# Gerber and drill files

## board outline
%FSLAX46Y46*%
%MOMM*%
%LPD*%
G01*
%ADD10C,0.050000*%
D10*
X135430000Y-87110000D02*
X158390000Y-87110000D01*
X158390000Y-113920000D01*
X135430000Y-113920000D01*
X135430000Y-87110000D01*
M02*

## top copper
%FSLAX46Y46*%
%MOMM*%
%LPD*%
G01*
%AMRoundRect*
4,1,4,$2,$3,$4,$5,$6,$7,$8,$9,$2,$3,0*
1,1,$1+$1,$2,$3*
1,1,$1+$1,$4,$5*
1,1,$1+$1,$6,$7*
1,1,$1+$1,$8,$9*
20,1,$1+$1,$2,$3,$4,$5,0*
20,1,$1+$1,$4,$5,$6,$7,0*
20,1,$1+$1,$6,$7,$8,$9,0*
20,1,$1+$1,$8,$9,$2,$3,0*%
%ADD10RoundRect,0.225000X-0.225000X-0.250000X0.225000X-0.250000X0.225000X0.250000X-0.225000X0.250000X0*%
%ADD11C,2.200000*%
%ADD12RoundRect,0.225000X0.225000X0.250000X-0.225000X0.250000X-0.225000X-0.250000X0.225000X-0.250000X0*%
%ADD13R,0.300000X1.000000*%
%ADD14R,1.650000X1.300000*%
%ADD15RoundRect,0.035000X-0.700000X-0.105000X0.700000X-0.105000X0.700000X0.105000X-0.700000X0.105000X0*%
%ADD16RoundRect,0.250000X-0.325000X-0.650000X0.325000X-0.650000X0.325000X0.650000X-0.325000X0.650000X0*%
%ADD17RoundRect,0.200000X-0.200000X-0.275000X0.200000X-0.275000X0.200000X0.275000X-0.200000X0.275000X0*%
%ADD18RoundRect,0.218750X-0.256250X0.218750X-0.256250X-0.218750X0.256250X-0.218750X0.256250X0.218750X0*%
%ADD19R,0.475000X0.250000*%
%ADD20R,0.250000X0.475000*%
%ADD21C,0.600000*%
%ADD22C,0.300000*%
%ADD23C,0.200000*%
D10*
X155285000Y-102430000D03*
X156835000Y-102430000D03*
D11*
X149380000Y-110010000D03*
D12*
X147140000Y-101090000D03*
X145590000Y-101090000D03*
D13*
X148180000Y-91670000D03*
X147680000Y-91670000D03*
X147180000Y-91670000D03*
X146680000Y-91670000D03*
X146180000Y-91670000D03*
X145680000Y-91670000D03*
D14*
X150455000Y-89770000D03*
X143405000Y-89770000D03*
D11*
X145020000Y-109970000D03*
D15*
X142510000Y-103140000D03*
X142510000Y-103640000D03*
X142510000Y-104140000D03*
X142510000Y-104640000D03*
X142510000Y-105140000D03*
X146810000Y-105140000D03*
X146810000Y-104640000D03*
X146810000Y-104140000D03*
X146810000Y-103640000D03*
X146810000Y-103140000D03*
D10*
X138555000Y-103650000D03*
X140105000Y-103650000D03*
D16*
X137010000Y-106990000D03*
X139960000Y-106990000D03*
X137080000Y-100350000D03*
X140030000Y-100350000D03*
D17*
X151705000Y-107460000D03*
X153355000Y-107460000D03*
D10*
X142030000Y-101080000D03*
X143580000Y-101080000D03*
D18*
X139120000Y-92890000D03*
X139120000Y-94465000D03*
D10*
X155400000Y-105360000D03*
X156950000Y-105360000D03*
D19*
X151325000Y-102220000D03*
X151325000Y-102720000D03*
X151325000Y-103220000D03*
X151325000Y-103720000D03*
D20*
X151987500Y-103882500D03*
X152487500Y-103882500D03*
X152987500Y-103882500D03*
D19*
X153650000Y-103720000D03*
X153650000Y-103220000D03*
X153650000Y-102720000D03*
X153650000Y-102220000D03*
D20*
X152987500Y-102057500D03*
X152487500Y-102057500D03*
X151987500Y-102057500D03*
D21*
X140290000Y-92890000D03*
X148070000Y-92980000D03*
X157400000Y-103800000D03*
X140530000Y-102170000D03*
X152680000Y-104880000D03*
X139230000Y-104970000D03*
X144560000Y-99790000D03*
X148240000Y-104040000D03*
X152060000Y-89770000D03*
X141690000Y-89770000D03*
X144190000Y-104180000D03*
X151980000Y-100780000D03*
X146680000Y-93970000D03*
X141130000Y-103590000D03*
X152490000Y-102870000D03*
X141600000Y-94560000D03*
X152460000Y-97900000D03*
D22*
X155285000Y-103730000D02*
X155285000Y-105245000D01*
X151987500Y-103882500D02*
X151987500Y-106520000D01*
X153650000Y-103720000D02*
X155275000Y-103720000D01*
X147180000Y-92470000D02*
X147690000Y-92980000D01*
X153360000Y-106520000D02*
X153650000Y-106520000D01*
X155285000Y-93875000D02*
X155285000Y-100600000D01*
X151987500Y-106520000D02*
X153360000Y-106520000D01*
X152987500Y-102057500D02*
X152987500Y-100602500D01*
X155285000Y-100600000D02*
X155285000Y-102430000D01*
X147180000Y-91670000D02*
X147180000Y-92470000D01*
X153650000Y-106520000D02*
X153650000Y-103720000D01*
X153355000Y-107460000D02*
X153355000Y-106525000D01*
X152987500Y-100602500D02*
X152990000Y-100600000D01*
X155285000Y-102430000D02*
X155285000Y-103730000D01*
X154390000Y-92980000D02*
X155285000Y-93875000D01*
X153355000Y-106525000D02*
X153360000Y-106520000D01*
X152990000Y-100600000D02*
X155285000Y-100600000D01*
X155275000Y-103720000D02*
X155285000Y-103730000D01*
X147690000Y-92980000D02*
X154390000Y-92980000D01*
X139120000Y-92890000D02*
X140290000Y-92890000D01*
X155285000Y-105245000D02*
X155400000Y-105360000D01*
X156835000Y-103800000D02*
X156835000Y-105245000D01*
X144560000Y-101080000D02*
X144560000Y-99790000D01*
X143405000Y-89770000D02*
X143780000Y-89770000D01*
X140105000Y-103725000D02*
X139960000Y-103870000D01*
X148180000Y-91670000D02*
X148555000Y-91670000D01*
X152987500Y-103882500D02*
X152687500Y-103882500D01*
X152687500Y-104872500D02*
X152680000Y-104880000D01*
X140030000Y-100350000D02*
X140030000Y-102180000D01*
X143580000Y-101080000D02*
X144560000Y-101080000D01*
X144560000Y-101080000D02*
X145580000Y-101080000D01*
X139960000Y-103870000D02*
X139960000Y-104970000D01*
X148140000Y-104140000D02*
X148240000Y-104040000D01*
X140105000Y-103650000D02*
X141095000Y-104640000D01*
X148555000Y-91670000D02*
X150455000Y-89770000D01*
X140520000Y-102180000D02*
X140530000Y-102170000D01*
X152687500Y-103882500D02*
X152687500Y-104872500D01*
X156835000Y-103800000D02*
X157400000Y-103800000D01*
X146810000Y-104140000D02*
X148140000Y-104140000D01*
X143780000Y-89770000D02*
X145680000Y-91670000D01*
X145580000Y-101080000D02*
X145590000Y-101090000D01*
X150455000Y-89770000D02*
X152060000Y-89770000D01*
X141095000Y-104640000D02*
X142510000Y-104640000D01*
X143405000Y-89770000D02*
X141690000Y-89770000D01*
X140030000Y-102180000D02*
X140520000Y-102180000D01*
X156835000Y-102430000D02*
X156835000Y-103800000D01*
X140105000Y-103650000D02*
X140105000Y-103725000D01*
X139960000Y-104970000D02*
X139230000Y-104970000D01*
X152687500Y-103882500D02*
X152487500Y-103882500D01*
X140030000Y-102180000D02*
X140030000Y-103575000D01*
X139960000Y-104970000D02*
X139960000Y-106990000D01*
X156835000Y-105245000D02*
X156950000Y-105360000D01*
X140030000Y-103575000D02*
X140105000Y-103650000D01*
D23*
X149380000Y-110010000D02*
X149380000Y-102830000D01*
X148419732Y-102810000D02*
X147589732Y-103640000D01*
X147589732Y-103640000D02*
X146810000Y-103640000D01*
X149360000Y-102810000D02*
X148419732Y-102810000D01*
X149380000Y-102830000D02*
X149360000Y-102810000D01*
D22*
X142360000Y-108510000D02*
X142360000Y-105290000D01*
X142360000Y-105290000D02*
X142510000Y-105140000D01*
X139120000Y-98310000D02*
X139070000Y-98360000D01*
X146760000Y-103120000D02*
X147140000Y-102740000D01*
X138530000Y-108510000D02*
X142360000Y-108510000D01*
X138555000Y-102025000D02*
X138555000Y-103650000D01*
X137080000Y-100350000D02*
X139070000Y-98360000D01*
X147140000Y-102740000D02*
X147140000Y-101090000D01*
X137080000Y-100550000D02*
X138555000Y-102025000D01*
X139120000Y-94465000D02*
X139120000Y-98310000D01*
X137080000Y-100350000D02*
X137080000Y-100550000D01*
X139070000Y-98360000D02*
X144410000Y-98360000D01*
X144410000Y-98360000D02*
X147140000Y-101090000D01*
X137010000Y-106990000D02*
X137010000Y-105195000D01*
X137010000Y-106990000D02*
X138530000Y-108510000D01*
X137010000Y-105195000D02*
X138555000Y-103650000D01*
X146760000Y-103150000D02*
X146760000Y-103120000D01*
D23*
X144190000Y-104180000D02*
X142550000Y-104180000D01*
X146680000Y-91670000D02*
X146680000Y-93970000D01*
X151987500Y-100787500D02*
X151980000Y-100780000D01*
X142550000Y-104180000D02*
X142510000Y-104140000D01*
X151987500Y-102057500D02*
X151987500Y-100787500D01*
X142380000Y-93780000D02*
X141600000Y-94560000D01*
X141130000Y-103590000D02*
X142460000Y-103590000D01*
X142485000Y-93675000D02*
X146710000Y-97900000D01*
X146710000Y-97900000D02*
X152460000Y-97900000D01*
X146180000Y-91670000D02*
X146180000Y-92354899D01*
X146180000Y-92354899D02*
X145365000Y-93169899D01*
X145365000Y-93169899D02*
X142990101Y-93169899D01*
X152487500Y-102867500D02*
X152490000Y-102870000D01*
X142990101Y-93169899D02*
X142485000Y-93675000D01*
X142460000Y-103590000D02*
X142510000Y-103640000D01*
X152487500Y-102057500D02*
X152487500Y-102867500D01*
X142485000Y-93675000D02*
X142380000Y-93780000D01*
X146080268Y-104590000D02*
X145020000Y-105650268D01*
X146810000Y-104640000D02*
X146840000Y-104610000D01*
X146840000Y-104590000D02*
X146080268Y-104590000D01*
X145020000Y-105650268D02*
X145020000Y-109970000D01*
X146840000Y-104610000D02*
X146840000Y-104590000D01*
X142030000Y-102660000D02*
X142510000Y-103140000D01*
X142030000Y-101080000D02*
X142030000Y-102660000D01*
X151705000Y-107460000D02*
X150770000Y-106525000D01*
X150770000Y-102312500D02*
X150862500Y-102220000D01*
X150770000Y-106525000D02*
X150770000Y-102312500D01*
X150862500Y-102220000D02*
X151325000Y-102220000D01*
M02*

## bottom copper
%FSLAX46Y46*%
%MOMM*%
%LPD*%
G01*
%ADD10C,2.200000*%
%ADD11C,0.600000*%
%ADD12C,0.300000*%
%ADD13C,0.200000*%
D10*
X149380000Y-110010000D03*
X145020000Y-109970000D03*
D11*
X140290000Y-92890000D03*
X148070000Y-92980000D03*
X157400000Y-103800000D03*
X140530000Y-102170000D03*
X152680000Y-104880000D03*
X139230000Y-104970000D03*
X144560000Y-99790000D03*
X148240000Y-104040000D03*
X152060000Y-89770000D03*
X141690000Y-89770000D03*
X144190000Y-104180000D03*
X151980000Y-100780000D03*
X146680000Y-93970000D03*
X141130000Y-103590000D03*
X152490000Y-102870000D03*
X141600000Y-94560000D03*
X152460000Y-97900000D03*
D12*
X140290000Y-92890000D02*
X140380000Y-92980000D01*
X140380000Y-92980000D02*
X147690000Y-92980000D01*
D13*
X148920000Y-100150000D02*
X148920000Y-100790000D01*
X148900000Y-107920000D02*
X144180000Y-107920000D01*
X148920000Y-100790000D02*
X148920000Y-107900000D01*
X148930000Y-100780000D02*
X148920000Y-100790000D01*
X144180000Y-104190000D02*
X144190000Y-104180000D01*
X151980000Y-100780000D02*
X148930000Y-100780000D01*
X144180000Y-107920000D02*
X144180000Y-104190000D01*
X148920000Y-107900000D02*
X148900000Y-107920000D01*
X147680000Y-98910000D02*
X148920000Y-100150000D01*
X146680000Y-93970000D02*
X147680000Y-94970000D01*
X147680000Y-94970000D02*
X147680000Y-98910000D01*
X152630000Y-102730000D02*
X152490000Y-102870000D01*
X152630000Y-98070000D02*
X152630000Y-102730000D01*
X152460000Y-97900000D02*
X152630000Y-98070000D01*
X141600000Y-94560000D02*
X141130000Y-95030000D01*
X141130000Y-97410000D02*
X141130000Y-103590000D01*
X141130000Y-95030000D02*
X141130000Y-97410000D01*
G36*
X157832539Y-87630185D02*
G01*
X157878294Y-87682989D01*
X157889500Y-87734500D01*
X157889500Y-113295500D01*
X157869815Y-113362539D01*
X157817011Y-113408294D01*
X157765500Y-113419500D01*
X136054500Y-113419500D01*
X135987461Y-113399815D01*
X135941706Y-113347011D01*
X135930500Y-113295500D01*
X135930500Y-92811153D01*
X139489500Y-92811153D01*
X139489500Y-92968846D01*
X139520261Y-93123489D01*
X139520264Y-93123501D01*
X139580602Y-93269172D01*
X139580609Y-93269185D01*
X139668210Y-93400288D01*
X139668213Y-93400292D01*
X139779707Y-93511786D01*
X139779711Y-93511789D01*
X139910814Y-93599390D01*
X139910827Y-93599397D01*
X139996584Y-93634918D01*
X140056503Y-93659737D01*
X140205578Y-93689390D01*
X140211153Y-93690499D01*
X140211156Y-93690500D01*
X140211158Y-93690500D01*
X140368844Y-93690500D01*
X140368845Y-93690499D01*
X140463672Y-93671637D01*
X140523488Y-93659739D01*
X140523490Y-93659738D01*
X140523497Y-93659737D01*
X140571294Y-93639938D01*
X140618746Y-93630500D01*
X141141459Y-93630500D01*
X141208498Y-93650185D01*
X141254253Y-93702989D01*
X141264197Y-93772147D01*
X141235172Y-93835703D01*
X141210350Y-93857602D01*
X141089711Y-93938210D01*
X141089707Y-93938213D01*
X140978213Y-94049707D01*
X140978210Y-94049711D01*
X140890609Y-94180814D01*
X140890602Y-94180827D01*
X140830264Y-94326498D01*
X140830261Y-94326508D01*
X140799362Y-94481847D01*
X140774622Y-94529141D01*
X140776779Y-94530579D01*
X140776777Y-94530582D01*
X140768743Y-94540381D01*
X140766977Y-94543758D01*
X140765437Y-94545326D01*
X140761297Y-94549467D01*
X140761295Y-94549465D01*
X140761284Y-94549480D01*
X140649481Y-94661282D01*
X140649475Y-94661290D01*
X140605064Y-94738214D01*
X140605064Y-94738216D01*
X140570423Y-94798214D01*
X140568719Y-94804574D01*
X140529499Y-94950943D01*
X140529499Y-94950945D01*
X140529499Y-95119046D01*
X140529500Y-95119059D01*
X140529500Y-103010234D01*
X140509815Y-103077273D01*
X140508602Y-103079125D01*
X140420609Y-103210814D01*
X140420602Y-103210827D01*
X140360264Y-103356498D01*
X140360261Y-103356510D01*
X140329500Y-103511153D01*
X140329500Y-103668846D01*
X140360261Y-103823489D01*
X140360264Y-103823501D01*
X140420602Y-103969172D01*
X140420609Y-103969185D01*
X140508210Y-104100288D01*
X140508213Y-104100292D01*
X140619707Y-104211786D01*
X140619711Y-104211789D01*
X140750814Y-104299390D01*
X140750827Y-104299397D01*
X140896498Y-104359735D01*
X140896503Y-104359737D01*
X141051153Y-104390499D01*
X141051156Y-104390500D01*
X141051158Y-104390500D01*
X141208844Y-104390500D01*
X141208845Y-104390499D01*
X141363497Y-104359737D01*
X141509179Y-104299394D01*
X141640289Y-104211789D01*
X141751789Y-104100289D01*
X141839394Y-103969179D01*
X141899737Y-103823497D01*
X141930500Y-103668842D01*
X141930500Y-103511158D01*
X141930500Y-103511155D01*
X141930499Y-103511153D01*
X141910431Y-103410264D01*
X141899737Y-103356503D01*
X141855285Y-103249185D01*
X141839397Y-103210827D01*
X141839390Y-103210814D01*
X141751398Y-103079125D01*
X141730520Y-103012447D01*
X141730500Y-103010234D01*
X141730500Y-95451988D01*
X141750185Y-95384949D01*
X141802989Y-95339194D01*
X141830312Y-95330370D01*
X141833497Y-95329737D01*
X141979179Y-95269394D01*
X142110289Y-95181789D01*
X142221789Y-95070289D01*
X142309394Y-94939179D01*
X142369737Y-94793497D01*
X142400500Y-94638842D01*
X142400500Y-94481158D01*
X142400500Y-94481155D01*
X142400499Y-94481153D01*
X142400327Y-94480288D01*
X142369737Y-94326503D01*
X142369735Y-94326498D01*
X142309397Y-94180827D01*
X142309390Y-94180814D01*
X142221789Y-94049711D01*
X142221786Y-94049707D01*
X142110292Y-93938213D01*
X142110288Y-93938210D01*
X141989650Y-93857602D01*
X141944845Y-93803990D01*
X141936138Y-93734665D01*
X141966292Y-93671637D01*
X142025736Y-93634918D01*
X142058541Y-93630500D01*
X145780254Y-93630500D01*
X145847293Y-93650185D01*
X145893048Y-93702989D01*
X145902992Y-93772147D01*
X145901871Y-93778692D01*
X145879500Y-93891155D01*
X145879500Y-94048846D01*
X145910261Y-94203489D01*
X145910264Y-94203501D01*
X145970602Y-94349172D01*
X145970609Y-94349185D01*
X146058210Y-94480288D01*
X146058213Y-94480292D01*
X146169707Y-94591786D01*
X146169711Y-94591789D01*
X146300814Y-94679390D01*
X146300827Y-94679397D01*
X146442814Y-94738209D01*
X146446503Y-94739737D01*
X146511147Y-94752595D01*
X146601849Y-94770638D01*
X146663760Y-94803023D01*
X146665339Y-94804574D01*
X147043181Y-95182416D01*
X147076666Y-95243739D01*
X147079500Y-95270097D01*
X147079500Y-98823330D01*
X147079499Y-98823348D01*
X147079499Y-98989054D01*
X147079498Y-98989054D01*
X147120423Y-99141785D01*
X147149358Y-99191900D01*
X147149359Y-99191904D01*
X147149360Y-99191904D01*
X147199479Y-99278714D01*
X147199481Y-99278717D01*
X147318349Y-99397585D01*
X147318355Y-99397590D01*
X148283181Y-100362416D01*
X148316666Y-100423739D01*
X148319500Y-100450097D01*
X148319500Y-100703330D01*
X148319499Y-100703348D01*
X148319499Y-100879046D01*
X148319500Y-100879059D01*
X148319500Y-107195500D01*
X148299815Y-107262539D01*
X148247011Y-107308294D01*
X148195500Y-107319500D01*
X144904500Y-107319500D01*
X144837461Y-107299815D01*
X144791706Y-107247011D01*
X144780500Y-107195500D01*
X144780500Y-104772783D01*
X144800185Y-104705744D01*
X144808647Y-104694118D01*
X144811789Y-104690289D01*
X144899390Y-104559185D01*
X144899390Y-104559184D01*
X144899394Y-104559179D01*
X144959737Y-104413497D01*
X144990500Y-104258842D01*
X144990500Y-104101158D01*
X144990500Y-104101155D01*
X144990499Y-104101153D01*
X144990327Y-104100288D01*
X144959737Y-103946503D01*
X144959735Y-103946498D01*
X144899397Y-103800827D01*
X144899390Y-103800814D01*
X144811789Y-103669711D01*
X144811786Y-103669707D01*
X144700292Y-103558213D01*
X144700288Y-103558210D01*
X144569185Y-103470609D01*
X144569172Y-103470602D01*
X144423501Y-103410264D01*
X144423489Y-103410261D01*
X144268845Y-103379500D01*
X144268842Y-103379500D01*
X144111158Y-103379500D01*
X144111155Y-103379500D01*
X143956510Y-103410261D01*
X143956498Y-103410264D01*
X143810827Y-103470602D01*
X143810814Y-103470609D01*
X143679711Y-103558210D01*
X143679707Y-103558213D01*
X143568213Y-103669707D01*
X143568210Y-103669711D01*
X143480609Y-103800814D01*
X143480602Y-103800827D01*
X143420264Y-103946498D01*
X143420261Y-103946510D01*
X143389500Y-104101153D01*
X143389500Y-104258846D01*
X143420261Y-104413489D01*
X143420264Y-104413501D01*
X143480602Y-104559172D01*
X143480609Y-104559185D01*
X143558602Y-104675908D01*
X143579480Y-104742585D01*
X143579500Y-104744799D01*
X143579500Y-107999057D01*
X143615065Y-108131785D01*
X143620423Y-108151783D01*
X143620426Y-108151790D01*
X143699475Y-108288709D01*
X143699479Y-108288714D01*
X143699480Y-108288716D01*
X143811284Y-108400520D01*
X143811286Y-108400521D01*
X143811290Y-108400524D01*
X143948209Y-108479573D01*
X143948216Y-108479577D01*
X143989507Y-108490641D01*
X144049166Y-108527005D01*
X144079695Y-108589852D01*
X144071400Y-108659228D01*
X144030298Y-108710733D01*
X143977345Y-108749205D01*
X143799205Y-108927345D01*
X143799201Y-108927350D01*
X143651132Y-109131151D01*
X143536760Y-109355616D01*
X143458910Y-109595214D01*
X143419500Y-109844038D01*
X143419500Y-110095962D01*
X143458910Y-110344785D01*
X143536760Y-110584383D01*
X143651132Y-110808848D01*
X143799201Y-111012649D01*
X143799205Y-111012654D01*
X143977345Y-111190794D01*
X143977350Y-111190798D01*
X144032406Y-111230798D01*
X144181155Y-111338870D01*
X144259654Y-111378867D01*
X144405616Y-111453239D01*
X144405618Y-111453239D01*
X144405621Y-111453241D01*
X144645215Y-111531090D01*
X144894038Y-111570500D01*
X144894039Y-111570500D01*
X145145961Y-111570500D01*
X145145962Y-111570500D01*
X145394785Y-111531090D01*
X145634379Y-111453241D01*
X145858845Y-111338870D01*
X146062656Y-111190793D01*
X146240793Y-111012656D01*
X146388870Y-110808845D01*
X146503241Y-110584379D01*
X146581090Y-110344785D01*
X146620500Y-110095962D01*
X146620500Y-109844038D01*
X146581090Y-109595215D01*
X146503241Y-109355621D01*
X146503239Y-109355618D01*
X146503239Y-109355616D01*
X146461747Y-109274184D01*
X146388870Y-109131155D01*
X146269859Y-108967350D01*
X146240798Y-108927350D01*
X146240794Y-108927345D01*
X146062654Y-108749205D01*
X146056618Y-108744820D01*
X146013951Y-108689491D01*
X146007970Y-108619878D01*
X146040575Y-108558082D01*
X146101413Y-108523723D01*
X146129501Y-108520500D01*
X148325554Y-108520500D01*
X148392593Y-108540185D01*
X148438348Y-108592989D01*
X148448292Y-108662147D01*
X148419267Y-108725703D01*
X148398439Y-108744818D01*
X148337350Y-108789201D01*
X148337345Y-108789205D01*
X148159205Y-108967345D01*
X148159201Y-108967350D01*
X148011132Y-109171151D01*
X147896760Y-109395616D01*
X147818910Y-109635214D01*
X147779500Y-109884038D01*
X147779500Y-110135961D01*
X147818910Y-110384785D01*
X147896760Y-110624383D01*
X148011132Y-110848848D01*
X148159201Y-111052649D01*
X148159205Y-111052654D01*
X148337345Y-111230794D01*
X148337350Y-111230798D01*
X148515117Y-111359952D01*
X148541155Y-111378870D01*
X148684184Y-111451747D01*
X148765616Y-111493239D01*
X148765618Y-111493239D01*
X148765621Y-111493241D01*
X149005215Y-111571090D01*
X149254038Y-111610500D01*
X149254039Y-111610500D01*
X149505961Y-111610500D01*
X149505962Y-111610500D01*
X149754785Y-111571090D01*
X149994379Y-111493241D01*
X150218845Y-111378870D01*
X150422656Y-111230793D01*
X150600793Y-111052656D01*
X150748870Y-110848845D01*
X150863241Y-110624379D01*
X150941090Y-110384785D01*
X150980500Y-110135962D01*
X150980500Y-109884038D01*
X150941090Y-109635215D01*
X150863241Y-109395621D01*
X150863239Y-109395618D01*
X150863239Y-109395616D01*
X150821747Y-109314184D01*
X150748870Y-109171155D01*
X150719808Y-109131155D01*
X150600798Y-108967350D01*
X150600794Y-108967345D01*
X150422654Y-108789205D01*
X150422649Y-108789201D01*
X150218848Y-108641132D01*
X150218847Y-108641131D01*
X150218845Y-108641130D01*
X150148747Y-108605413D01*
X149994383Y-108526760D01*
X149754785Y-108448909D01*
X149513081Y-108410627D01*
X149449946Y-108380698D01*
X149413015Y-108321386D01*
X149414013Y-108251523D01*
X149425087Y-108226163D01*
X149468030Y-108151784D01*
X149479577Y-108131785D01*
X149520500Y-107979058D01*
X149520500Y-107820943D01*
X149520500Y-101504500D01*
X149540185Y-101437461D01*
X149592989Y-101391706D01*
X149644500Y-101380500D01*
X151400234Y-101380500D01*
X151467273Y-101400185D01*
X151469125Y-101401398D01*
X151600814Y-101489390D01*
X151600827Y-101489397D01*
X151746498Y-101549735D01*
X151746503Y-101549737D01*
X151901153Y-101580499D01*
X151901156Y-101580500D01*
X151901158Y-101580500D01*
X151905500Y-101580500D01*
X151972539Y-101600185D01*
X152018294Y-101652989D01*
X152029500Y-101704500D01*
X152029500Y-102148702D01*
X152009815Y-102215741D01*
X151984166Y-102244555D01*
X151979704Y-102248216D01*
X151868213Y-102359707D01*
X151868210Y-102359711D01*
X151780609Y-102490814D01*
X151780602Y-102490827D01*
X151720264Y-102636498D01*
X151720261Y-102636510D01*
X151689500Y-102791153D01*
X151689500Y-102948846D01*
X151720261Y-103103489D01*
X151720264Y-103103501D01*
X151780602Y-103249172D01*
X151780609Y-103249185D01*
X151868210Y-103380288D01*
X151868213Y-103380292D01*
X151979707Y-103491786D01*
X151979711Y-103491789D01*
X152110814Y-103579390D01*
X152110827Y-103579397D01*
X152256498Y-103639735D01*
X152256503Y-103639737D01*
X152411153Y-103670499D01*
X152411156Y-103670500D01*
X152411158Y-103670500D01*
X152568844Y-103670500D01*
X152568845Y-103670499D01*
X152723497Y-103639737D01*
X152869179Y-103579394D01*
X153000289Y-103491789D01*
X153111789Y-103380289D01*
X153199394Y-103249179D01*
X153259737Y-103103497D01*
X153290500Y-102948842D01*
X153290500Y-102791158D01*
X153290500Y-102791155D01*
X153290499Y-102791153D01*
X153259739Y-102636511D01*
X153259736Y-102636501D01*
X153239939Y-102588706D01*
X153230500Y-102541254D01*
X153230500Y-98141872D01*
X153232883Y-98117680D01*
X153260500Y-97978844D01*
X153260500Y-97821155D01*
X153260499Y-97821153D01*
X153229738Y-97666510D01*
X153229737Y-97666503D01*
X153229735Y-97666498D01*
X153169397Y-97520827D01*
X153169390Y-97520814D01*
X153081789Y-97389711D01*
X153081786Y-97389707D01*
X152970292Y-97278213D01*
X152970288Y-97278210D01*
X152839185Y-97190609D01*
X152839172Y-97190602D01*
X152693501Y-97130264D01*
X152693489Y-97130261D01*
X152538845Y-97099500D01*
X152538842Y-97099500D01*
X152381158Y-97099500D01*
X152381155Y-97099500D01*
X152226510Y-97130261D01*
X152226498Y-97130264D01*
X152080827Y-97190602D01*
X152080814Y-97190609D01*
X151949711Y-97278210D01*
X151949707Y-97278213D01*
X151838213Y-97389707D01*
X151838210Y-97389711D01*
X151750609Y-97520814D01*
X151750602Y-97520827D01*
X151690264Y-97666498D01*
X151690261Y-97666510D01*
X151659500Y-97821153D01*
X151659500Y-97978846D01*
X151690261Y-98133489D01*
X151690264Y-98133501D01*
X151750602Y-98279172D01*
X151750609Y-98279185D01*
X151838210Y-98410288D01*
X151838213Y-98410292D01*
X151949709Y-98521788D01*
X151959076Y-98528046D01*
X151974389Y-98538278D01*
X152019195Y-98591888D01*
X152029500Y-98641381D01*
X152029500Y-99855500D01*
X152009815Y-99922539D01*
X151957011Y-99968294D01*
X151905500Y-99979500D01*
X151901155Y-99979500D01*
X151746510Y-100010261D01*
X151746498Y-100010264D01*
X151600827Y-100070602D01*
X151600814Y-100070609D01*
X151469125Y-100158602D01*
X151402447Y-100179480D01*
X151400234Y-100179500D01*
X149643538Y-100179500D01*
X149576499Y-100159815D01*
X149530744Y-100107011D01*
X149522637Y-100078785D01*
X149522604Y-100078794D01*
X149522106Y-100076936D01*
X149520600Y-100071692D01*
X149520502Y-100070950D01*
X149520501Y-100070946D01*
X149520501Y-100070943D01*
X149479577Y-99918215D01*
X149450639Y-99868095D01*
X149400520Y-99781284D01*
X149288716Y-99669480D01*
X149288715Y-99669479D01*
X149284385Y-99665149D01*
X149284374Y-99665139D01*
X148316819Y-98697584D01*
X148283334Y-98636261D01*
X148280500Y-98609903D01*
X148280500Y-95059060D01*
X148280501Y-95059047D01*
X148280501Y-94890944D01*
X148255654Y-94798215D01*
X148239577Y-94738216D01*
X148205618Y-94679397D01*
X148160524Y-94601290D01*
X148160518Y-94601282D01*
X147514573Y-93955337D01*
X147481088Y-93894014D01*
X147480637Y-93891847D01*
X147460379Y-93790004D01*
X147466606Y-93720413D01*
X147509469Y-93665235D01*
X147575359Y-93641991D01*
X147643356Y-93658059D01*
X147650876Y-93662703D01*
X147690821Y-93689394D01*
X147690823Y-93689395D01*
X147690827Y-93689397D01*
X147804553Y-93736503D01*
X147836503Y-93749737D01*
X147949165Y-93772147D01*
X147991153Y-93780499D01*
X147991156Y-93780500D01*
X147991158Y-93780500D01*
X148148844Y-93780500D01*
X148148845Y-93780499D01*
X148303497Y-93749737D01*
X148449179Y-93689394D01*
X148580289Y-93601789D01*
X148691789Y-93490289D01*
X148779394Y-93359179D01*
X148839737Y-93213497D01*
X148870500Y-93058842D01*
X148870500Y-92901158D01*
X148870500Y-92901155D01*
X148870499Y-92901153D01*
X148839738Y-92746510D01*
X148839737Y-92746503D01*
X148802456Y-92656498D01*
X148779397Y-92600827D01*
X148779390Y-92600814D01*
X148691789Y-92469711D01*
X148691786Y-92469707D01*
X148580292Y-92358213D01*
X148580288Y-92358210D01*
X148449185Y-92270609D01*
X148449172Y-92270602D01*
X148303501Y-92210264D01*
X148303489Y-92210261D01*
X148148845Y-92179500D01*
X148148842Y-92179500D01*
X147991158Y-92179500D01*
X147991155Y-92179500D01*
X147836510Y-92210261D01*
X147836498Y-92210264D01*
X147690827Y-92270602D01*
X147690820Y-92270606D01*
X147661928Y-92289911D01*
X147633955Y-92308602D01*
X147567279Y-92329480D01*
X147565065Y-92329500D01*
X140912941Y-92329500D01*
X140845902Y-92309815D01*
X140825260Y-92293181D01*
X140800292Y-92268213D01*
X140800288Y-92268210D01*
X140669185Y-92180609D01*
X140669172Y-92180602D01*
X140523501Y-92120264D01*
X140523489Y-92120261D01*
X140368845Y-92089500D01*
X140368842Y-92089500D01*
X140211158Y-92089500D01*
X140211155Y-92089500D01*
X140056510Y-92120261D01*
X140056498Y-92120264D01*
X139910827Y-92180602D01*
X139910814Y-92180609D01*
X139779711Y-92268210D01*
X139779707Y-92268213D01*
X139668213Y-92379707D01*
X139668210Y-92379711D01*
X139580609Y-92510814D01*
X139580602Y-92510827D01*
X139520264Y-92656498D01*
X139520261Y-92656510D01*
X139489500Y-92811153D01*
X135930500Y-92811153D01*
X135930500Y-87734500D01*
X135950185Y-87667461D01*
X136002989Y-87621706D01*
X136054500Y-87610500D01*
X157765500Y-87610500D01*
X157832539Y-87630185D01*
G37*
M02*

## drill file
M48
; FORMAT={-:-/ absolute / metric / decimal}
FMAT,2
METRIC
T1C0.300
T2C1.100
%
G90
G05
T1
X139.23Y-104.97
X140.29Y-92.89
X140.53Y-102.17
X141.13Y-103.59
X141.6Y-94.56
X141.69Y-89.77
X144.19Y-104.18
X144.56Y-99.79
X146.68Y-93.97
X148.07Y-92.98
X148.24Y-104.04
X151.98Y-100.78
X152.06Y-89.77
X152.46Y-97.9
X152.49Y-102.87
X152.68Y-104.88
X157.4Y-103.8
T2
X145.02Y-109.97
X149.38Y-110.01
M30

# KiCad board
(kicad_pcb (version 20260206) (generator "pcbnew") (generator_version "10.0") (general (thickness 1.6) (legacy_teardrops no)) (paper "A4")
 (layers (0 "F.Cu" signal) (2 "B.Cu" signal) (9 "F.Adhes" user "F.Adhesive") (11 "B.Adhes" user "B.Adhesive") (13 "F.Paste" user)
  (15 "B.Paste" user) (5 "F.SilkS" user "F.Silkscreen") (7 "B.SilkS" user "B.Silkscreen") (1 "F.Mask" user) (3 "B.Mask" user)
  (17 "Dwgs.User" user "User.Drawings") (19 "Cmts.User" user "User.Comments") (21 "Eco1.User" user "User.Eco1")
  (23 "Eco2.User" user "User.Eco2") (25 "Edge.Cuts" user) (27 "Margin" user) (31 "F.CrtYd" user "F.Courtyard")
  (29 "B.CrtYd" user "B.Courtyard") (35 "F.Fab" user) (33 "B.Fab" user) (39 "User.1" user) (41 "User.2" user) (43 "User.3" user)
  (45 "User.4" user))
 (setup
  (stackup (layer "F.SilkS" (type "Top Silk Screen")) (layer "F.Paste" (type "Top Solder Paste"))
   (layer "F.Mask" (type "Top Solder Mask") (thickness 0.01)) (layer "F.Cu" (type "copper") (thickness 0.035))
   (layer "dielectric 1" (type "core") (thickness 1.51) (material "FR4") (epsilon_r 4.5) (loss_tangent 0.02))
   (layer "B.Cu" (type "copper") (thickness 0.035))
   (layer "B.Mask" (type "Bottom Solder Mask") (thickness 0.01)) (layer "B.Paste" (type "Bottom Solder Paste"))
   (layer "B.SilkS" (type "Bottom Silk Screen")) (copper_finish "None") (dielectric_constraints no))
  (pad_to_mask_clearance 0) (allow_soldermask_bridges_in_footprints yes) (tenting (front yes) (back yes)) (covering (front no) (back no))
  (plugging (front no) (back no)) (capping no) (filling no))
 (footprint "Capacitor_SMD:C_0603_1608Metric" (layer "F.Cu") (at 156.06 102.43)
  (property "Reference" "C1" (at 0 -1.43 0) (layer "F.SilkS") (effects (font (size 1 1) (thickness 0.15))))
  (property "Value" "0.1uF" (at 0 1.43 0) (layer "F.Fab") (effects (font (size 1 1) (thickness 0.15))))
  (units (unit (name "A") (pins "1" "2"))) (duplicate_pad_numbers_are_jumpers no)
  (pad "1" smd roundrect (at -0.775 0) (size 0.9 0.95) (layers "F.Cu" "F.Mask" "F.Paste") (roundrect_rratio 0.25) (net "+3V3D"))
  (pad "2" smd roundrect (at 0.775 0) (size 0.9 0.95) (layers "F.Cu" "F.Mask" "F.Paste") (roundrect_rratio 0.25) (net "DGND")))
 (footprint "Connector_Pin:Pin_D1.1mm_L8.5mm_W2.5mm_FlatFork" (layer "F.Cu") (at 149.38 110.01)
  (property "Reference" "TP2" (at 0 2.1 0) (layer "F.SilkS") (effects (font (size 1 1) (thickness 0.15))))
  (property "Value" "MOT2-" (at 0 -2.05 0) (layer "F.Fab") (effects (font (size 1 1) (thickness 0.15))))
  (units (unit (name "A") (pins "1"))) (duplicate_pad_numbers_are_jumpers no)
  (pad "1" thru_hole circle (at 0 0) (size 2.2 2.2) (drill 1.1) (layers "*.Cu" "*.Mask") (remove_unused_layers no) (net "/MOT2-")))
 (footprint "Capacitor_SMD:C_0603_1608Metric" (layer "F.Cu") (at 146.365 101.09 180)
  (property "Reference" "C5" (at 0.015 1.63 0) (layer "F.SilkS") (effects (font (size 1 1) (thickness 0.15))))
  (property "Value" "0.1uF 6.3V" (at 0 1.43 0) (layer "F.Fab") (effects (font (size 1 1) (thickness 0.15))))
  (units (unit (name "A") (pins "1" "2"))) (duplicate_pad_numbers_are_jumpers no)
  (pad "1" smd roundrect (at -0.775 0 180) (size 0.9 0.95) (layers "F.Cu" "F.Mask" "F.Paste") (roundrect_rratio 0.25) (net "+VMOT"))
  (pad "2" smd roundrect (at 0.775 0 180) (size 0.9 0.95) (layers "F.Cu" "F.Mask" "F.Paste") (roundrect_rratio 0.25) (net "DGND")))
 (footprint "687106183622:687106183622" (layer "F.Cu") (at 146.93 89.37 180)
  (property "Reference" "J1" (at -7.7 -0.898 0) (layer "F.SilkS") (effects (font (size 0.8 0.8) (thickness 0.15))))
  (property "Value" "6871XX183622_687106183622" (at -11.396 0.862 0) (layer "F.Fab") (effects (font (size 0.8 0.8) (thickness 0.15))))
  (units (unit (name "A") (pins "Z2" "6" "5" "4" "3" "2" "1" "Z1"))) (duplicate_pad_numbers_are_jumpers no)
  (pad "1" smd rect (at -1.25 -2.3 180) (size 0.3 1) (layers "F.Cu" "F.Mask" "F.Paste") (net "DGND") (solder_mask_margin 0.102))
  (pad "2" smd rect (at -0.75 -2.3 180) (size 0.3 1) (layers "F.Cu" "F.Mask" "F.Paste") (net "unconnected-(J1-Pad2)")
   (solder_mask_margin 0.102))
  (pad "3" smd rect (at -0.25 -2.3 180) (size 0.3 1) (layers "F.Cu" "F.Mask" "F.Paste") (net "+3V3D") (solder_mask_margin 0.102))
  (pad "4" smd rect (at 0.25 -2.3 180) (size 0.3 1) (layers "F.Cu" "F.Mask" "F.Paste") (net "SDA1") (solder_mask_margin 0.102))
  (pad "5" smd rect (at 0.75 -2.3 180) (size 0.3 1) (layers "F.Cu" "F.Mask" "F.Paste") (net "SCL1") (solder_mask_margin 0.102))
  (pad "6" smd rect (at 1.25 -2.3 180) (size 0.3 1) (layers "F.Cu" "F.Mask" "F.Paste") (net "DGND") (solder_mask_margin 0.102))
  (pad "Z1" smd rect (at -3.525 -0.4 180) (size 1.65 1.3) (layers "F.Cu" "F.Mask" "F.Paste") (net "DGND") (solder_mask_margin 0.102))
  (pad "Z2" smd rect (at 3.525 -0.4 180) (size 1.65 1.3) (layers "F.Cu" "F.Mask" "F.Paste") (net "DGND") (solder_mask_margin 0.102)))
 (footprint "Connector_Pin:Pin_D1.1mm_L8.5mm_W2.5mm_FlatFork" (layer "F.Cu") (at 145.02 109.97)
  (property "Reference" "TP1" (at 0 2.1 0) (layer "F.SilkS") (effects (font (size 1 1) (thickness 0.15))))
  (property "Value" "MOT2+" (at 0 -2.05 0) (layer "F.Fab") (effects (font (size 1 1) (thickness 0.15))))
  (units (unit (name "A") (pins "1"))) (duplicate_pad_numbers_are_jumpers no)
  (pad "1" thru_hole circle (at 0 0) (size 2.2 2.2) (drill 1.1) (layers "*.Cu" "*.Mask") (remove_unused_layers no) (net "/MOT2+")))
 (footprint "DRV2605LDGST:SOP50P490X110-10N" (layer "F.Cu") (at 144.66 104.14)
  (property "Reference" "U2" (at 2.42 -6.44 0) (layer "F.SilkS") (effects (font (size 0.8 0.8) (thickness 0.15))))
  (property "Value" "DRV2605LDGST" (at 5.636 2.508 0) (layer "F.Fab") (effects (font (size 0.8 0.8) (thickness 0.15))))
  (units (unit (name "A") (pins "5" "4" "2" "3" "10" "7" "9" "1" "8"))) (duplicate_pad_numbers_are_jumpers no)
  (pad "1" smd roundrect (at -2.15 -1) (size 1.47 0.28) (layers "F.Cu" "F.Mask" "F.Paste") (roundrect_rratio 0.125) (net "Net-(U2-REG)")
   (solder_mask_margin 0.102))
  (pad "2" smd roundrect (at -2.15 -0.5) (size 1.47 0.28) (layers "F.Cu" "F.Mask" "F.Paste") (roundrect_rratio 0.125) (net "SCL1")
   (solder_mask_margin 0.102))
  (pad "3" smd roundrect (at -2.15 0) (size 1.47 0.28) (layers "F.Cu" "F.Mask" "F.Paste") (roundrect_rratio 0.125) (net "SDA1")
   (solder_mask_margin 0.102))
  (pad "4" smd roundrect (at -2.15 0.5) (size 1.47 0.28) (layers "F.Cu" "F.Mask" "F.Paste") (roundrect_rratio 0.125) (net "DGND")
   (solder_mask_margin 0.102))
  (pad "5" smd roundrect (at -2.15 1) (size 1.47 0.28) (layers "F.Cu" "F.Mask" "F.Paste") (roundrect_rratio 0.125) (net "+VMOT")
   (solder_mask_margin 0.102))
  (pad "6" smd roundrect (at 2.15 1) (size 1.47 0.28) (layers "F.Cu" "F.Mask" "F.Paste") (roundrect_rratio 0.125) (solder_mask_margin 0.102))
  (pad "7" smd roundrect (at 2.15 0.5) (size 1.47 0.28) (layers "F.Cu" "F.Mask" "F.Paste") (roundrect_rratio 0.125) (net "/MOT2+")
   (solder_mask_margin 0.102))
  (pad "8" smd roundrect (at 2.15 0) (size 1.47 0.28) (layers "F.Cu" "F.Mask" "F.Paste") (roundrect_rratio 0.125) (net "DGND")
   (solder_mask_margin 0.102))
  (pad "9" smd roundrect (at 2.15 -0.5) (size 1.47 0.28) (layers "F.Cu" "F.Mask" "F.Paste") (roundrect_rratio 0.125) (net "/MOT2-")
   (solder_mask_margin 0.102))
  (pad "10" smd roundrect (at 2.15 -1) (size 1.47 0.28) (layers "F.Cu" "F.Mask" "F.Paste") (roundrect_rratio 0.125) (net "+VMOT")
   (solder_mask_margin 0.102)))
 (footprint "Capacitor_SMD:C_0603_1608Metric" (layer "F.Cu") (at 139.33 103.65)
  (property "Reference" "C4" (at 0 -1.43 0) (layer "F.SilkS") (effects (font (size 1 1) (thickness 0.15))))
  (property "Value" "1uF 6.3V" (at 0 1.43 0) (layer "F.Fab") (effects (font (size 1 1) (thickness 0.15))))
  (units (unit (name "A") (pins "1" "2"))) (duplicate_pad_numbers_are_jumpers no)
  (pad "1" smd roundrect (at -0.775 0) (size 0.9 0.95) (layers "F.Cu" "F.Mask" "F.Paste") (roundrect_rratio 0.25) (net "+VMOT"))
  (pad "2" smd roundrect (at 0.775 0) (size 0.9 0.95) (layers "F.Cu" "F.Mask" "F.Paste") (roundrect_rratio 0.25) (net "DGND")))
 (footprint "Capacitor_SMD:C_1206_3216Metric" (layer "F.Cu") (at 138.485 106.99)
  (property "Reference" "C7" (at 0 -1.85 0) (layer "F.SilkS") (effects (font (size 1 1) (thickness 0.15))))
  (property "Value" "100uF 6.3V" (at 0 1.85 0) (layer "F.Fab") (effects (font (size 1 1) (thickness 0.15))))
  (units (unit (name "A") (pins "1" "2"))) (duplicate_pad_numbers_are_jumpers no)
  (pad "1" smd roundrect (at -1.475 0) (size 1.15 1.8) (layers "F.Cu" "F.Mask" "F.Paste") (roundrect_rratio 0.217391) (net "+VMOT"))
  (pad "2" smd roundrect (at 1.475 0) (size 1.15 1.8) (layers "F.Cu" "F.Mask" "F.Paste") (roundrect_rratio 0.217391) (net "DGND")))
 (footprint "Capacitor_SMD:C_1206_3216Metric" (layer "F.Cu") (at 138.555 100.35)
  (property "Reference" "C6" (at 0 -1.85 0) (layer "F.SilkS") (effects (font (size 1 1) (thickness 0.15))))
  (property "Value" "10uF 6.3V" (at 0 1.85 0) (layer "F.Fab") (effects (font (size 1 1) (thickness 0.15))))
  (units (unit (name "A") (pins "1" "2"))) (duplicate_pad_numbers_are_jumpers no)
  (pad "1" smd roundrect (at -1.475 0) (size 1.15 1.8) (layers "F.Cu" "F.Mask" "F.Paste") (roundrect_rratio 0.217391) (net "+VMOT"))
  (pad "2" smd roundrect (at 1.475 0) (size 1.15 1.8) (layers "F.Cu" "F.Mask" "F.Paste") (roundrect_rratio 0.217391) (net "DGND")))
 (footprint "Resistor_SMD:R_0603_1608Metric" (layer "F.Cu") (at 152.53 107.46)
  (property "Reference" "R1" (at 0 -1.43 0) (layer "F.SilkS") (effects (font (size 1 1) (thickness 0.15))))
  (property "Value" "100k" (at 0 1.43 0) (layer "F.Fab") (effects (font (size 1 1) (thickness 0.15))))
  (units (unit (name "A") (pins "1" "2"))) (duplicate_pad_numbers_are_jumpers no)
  (pad "1" smd roundrect (at -0.825 0) (size 0.8 0.95) (layers "F.Cu" "F.Mask" "F.Paste") (roundrect_rratio 0.25) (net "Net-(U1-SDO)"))
  (pad "2" smd roundrect (at 0.825 0) (size 0.8 0.95) (layers "F.Cu" "F.Mask" "F.Paste") (roundrect_rratio 0.25) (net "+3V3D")))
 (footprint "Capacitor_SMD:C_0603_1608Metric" (layer "F.Cu") (at 142.805 101.08)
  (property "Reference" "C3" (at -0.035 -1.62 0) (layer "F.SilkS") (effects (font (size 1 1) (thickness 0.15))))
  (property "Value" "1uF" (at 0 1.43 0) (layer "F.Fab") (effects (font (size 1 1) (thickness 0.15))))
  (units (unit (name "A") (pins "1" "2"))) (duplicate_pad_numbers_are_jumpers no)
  (pad "1" smd roundrect (at -0.775 0) (size 0.9 0.95) (layers "F.Cu" "F.Mask" "F.Paste") (roundrect_rratio 0.25) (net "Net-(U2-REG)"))
  (pad "2" smd roundrect (at 0.775 0) (size 0.9 0.95) (layers "F.Cu" "F.Mask" "F.Paste") (roundrect_rratio 0.25) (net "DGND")))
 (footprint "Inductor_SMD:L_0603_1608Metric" (layer "F.Cu") (at 139.12 93.6775 -90)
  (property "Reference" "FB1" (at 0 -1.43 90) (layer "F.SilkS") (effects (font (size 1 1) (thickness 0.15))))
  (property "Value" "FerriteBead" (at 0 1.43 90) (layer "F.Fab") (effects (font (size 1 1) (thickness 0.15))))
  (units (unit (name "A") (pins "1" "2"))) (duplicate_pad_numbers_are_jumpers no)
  (pad "1" smd roundrect (at -0.7875 0 270) (size 0.875 0.95) (layers "F.Cu" "F.Mask" "F.Paste") (roundrect_rratio 0.25) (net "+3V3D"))
  (pad "2" smd roundrect (at 0.7875 0 270) (size 0.875 0.95) (layers "F.Cu" "F.Mask" "F.Paste") (roundrect_rratio 0.25) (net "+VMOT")))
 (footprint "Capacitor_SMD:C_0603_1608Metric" (layer "F.Cu") (at 156.175 105.36)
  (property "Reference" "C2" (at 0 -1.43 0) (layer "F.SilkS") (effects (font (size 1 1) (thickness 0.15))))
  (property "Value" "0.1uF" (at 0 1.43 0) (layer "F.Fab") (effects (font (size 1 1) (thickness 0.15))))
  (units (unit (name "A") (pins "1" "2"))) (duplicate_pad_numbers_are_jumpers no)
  (pad "1" smd roundrect (at -0.775 0) (size 0.9 0.95) (layers "F.Cu" "F.Mask" "F.Paste") (roundrect_rratio 0.25) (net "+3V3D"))
  (pad "2" smd roundrect (at 0.775 0) (size 0.9 0.95) (layers "F.Cu" "F.Mask" "F.Paste") (roundrect_rratio 0.25) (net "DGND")))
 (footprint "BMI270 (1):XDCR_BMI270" (layer "F.Cu") (at 152.4875 102.97)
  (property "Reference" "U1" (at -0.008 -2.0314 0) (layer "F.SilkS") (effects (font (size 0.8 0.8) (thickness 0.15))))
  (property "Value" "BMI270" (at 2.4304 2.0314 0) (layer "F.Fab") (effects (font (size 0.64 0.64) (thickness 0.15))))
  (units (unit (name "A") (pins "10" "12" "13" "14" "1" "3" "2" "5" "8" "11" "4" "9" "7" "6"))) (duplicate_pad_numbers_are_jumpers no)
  (pad "1" smd rect (at -1.1625 -0.75) (size 0.475 0.25) (layers "F.Cu" "F.Mask" "F.Paste") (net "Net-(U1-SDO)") (solder_mask_margin 0.102))
  (pad "2" smd rect (at -1.1625 -0.25) (size 0.475 0.25) (layers "F.Cu" "F.Mask" "F.Paste") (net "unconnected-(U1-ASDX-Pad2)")
   (solder_mask_margin 0.102))
  (pad "3" smd rect (at -1.1625 0.25) (size 0.475 0.25) (layers "F.Cu" "F.Mask" "F.Paste") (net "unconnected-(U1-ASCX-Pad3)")
   (solder_mask_margin 0.102))
  (pad "4" smd rect (at -1.1625 0.75) (size 0.475 0.25) (layers "F.Cu" "F.Mask" "F.Paste") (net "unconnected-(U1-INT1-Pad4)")
   (solder_mask_margin 0.102))
  (pad "5" smd rect (at -0.5 0.9125) (size 0.25 0.475) (layers "F.Cu" "F.Mask" "F.Paste") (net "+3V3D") (solder_mask_margin 0.102))
  (pad "6" smd rect (at 0 0.9125) (size 0.25 0.475) (layers "F.Cu" "F.Mask" "F.Paste") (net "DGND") (solder_mask_margin 0.102))
  (pad "7" smd rect (at 0.5 0.9125) (size 0.25 0.475) (layers "F.Cu" "F.Mask" "F.Paste") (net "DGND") (solder_mask_margin 0.102))
  (pad "8" smd rect (at 1.1625 0.75) (size 0.475 0.25) (layers "F.Cu" "F.Mask" "F.Paste") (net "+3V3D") (solder_mask_margin 0.102))
  (pad "9" smd rect (at 1.1625 0.25) (size 0.475 0.25) (layers "F.Cu" "F.Mask" "F.Paste") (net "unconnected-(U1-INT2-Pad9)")
   (solder_mask_margin 0.102))
  (pad "10" smd rect (at 1.1625 -0.25) (size 0.475 0.25) (layers "F.Cu" "F.Mask" "F.Paste") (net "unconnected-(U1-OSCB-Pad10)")
   (solder_mask_margin 0.102))
  (pad "11" smd rect (at 1.1625 -0.75) (size 0.475 0.25) (layers "F.Cu" "F.Mask" "F.Paste") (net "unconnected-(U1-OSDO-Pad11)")
   (solder_mask_margin 0.102))
  (pad "12" smd rect (at 0.5 -0.9125) (size 0.25 0.475) (layers "F.Cu" "F.Mask" "F.Paste") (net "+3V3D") (solder_mask_margin 0.102))
  (pad "13" smd rect (at 0 -0.9125) (size 0.25 0.475) (layers "F.Cu" "F.Mask" "F.Paste") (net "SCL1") (solder_mask_margin 0.102))
  (pad "14" smd rect (at -0.5 -0.9125) (size 0.25 0.475) (layers "F.Cu" "F.Mask" "F.Paste") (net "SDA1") (solder_mask_margin 0.102)))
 (gr_rect (start 135.43 87.11) (end 158.39 113.92) (stroke (width 0.05) (type solid)) (fill no) (layer "Edge.Cuts"))
 (segment (start 155.285 103.73) (end 155.285 105.245) (width 0.3) (layer "F.Cu") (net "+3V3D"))
 (segment (start 151.9875 103.8825) (end 151.9875 106.52) (width 0.3) (layer "F.Cu") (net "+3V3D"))
 (segment (start 153.65 103.72) (end 155.275 103.72) (width 0.3) (layer "F.Cu") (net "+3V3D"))
 (segment (start 147.18 92.47) (end 147.69 92.98) (width 0.3) (layer "F.Cu") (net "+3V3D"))
 (segment (start 153.36 106.52) (end 153.65 106.52) (width 0.3) (layer "F.Cu") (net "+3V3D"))
 (segment (start 155.285 93.875) (end 155.285 100.6) (width 0.3) (layer "F.Cu") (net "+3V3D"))
 (segment (start 151.9875 106.52) (end 153.36 106.52) (width 0.3) (layer "F.Cu") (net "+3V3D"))
 (segment (start 152.9875 102.0575) (end 152.9875 100.6025) (width 0.3) (layer "F.Cu") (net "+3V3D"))
 (segment (start 155.285 100.6) (end 155.285 102.43) (width 0.3) (layer "F.Cu") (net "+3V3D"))
 (segment (start 147.18 91.67) (end 147.18 92.47) (width 0.3) (layer "F.Cu") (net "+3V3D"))
 (segment (start 153.65 106.52) (end 153.65 103.72) (width 0.3) (layer "F.Cu") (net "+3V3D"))
 (segment (start 153.355 107.46) (end 153.355 106.525) (width 0.3) (layer "F.Cu") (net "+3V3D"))
 (segment (start 152.9875 100.6025) (end 152.99 100.6) (width 0.3) (layer "F.Cu") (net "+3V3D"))
 (segment (start 155.285 102.43) (end 155.285 103.73) (width 0.3) (layer "F.Cu") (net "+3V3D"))
 (segment (start 154.39 92.98) (end 155.285 93.875) (width 0.3) (layer "F.Cu") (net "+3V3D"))
 (segment (start 153.355 106.525) (end 153.36 106.52) (width 0.3) (layer "F.Cu") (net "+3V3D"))
 (segment (start 152.99 100.6) (end 155.285 100.6) (width 0.3) (layer "F.Cu") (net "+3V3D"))
 (segment (start 155.275 103.72) (end 155.285 103.73) (width 0.3) (layer "F.Cu") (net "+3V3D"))
 (segment (start 147.69 92.98) (end 154.39 92.98) (width 0.3) (layer "F.Cu") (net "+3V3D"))
 (segment (start 139.12 92.89) (end 140.29 92.89) (width 0.3) (layer "F.Cu") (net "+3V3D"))
 (segment (start 155.285 105.245) (end 155.4 105.36) (width 0.3) (layer "F.Cu") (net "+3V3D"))
 (via (at 140.29 92.89) (size 0.6) (drill 0.3) (layers "F.Cu" "B.Cu") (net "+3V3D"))
 (via (at 148.07 92.98) (size 0.6) (drill 0.3) (layers "F.Cu" "B.Cu") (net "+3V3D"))
 (segment (start 140.29 92.89) (end 140.38 92.98) (width 0.3) (layer "B.Cu") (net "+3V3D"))
 (segment (start 140.38 92.98) (end 147.69 92.98) (width 0.3) (layer "B.Cu") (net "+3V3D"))
 (segment (start 156.835 103.8) (end 156.835 105.245) (width 0.3) (layer "F.Cu") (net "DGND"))
 (segment (start 144.56 101.08) (end 144.56 99.79) (width 0.3) (layer "F.Cu") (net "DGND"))
 (segment (start 143.405 89.77) (end 143.78 89.77) (width 0.3) (layer "F.Cu") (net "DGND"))
 (segment (start 140.105 103.725) (end 139.96 103.87) (width 0.3) (layer "F.Cu") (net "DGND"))
 (segment (start 148.18 91.67) (end 148.555 91.67) (width 0.3) (layer "F.Cu") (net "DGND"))
 (segment (start 152.9875 103.8825) (end 152.6875 103.8825) (width 0.3) (layer "F.Cu") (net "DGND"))
 (segment (start 152.6875 104.8725) (end 152.68 104.88) (width 0.3) (layer "F.Cu") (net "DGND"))
 (segment (start 140.03 100.35) (end 140.03 102.18) (width 0.3) (layer "F.Cu") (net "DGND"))
 (segment (start 143.58 101.08) (end 144.56 101.08) (width 0.3) (layer "F.Cu") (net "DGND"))
 (segment (start 144.56 101.08) (end 145.58 101.08) (width 0.3) (layer "F.Cu") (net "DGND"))
 (segment (start 139.96 103.87) (end 139.96 104.97) (width 0.3) (layer "F.Cu") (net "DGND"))
 (segment (start 148.14 104.14) (end 148.24 104.04) (width 0.3) (layer "F.Cu") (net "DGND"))
 (segment (start 140.105 103.65) (end 141.095 104.64) (width 0.3) (layer "F.Cu") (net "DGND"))
 (segment (start 148.555 91.67) (end 150.455 89.77) (width 0.3) (layer "F.Cu") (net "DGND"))
 (segment (start 140.52 102.18) (end 140.53 102.17) (width 0.3) (layer "F.Cu") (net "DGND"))
 (segment (start 152.6875 103.8825) (end 152.6875 104.8725) (width 0.3) (layer "F.Cu") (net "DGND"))
 (segment (start 156.835 103.8) (end 157.4 103.8) (width 0.3) (layer "F.Cu") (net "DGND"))
 (segment (start 146.81 104.14) (end 148.14 104.14) (width 0.3) (layer "F.Cu") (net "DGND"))
 (segment (start 143.78 89.77) (end 145.68 91.67) (width 0.3) (layer "F.Cu") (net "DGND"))
 (segment (start 145.58 101.08) (end 145.59 101.09) (width 0.3) (layer "F.Cu") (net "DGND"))
 (segment (start 150.455 89.77) (end 152.06 89.77) (width 0.3) (layer "F.Cu") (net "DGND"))
 (segment (start 141.095 104.64) (end 142.51 104.64) (width 0.3) (layer "F.Cu") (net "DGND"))
 (segment (start 143.405 89.77) (end 141.69 89.77) (width 0.3) (layer "F.Cu") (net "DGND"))
 (segment (start 140.03 102.18) (end 140.52 102.18) (width 0.3) (layer "F.Cu") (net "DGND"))
 (segment (start 156.835 102.43) (end 156.835 103.8) (width 0.3) (layer "F.Cu") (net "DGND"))
 (segment (start 140.105 103.65) (end 140.105 103.725) (width 0.3) (layer "F.Cu") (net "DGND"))
 (segment (start 139.96 104.97) (end 139.23 104.97) (width 0.3) (layer "F.Cu") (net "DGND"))
 (segment (start 152.6875 103.8825) (end 152.4875 103.8825) (width 0.3) (layer "F.Cu") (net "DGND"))
 (segment (start 140.03 102.18) (end 140.03 103.575) (width 0.3) (layer "F.Cu") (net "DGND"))
 (segment (start 139.96 104.97) (end 139.96 106.99) (width 0.3) (layer "F.Cu") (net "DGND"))
 (segment (start 156.835 105.245) (end 156.95 105.36) (width 0.3) (layer "F.Cu") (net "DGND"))
 (segment (start 140.03 103.575) (end 140.105 103.65) (width 0.3) (layer "F.Cu") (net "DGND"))
 (via (at 157.4 103.8) (size 0.6) (drill 0.3) (layers "F.Cu" "B.Cu") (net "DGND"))
 (via (at 140.53 102.17) (size 0.6) (drill 0.3) (layers "F.Cu" "B.Cu") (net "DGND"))
 (via (at 152.68 104.88) (size 0.6) (drill 0.3) (layers "F.Cu" "B.Cu") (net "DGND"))
 (via (at 139.23 104.97) (size 0.6) (drill 0.3) (layers "F.Cu" "B.Cu") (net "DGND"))
 (via (at 144.56 99.79) (size 0.6) (drill 0.3) (layers "F.Cu" "B.Cu") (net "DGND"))
 (via (at 148.24 104.04) (size 0.6) (drill 0.3) (layers "F.Cu" "B.Cu") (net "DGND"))
 (via (at 152.06 89.77) (size 0.6) (drill 0.3) (layers "F.Cu" "B.Cu") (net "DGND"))
 (via (at 141.69 89.77) (size 0.6) (drill 0.3) (layers "F.Cu" "B.Cu") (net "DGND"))
 (segment (start 149.38 110.01) (end 149.38 102.83) (width 0.2) (layer "F.Cu") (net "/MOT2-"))
 (segment (start 148.419732 102.81) (end 147.589732 103.64) (width 0.2) (layer "F.Cu") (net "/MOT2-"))
 (segment (start 147.589732 103.64) (end 146.81 103.64) (width 0.2) (layer "F.Cu") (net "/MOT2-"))
 (segment (start 149.36 102.81) (end 148.419732 102.81) (width 0.2) (layer "F.Cu") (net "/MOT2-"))
 (segment (start 149.38 102.83) (end 149.36 102.81) (width 0.2) (layer "F.Cu") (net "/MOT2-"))
 (segment (start 142.36 108.51) (end 142.36 105.29) (width 0.3) (layer "F.Cu") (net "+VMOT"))
 (segment (start 142.36 105.29) (end 142.51 105.14) (width 0.3) (layer "F.Cu") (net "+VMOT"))
 (segment (start 139.12 98.31) (end 139.07 98.36) (width 0.3) (layer "F.Cu") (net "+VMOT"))
 (segment (start 146.76 103.12) (end 147.14 102.74) (width 0.3) (layer "F.Cu") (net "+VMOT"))
 (segment (start 138.53 108.51) (end 142.36 108.51) (width 0.3) (layer "F.Cu") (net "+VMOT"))
 (segment (start 138.555 102.025) (end 138.555 103.65) (width 0.3) (layer "F.Cu") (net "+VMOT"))
 (segment (start 137.08 100.35) (end 139.07 98.36) (width 0.3) (layer "F.Cu") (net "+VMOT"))
 (segment (start 147.14 102.74) (end 147.14 101.09) (width 0.3) (layer "F.Cu") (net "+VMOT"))
 (segment (start 137.08 100.55) (end 138.555 102.025) (width 0.3) (layer "F.Cu") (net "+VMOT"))
 (segment (start 139.12 94.465) (end 139.12 98.31) (width 0.3) (layer "F.Cu") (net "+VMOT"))
 (segment (start 137.08 100.35) (end 137.08 100.55) (width 0.3) (layer "F.Cu") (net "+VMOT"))
 (segment (start 139.07 98.36) (end 144.41 98.36) (width 0.3) (layer "F.Cu") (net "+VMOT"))
 (segment (start 144.41 98.36) (end 147.14 101.09) (width 0.3) (layer "F.Cu") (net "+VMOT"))
 (segment (start 137.01 106.99) (end 137.01 105.195) (width 0.3) (layer "F.Cu") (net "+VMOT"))
 (segment (start 137.01 106.99) (end 138.53 108.51) (width 0.3) (layer "F.Cu") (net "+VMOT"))
 (segment (start 137.01 105.195) (end 138.555 103.65) (width 0.3) (layer "F.Cu") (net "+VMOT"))
 (segment (start 146.76 103.15) (end 146.76 103.12) (width 0.3) (layer "F.Cu") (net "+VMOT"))
 (segment (start 144.19 104.18) (end 142.55 104.18) (width 0.2) (layer "F.Cu") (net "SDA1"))
 (segment (start 146.68 91.67) (end 146.68 93.97) (width 0.2) (layer "F.Cu") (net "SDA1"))
 (segment (start 151.9875 100.7875) (end 151.98 100.78) (width 0.2) (layer "F.Cu") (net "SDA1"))
 (segment (start 142.55 104.18) (end 142.51 104.14) (width 0.2) (layer "F.Cu") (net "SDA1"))
 (segment (start 151.9875 102.0575) (end 151.9875 100.7875) (width 0.2) (layer "F.Cu") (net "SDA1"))
 (via (at 144.19 104.18) (size 0.6) (drill 0.3) (layers "F.Cu" "B.Cu") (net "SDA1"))
 (via (at 151.98 100.78) (size 0.6) (drill 0.3) (layers "F.Cu" "B.Cu") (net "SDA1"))
 (via (at 146.68 93.97) (size 0.6) (drill 0.3) (layers "F.Cu" "B.Cu") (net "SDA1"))
 (segment (start 148.92 100.15) (end 148.92 100.79) (width 0.2) (layer "B.Cu") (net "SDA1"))
 (segment (start 148.9 107.92) (end 144.18 107.92) (width 0.2) (layer "B.Cu") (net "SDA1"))
 (segment (start 148.92 100.79) (end 148.92 107.9) (width 0.2) (layer "B.Cu") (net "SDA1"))
 (segment (start 148.93 100.78) (end 148.92 100.79) (width 0.2) (layer "B.Cu") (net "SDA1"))
 (segment (start 144.18 104.19) (end 144.19 104.18) (width 0.2) (layer "B.Cu") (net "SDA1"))
 (segment (start 151.98 100.78) (end 148.93 100.78) (width 0.2) (layer "B.Cu") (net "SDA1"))
 (segment (start 144.18 107.92) (end 144.18 104.19) (width 0.2) (layer "B.Cu") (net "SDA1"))
 (segment (start 148.92 107.9) (end 148.9 107.92) (width 0.2) (layer "B.Cu") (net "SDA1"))
 (segment (start 147.68 98.91) (end 148.92 100.15) (width 0.2) (layer "B.Cu") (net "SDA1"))
 (segment (start 146.68 93.97) (end 147.68 94.97) (width 0.2) (layer "B.Cu") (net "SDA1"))
 (segment (start 147.68 94.97) (end 147.68 98.91) (width 0.2) (layer "B.Cu") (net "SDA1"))
 (segment (start 142.38 93.78) (end 141.6 94.56) (width 0.2) (layer "F.Cu") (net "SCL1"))
 (segment (start 141.13 103.59) (end 142.46 103.59) (width 0.2) (layer "F.Cu") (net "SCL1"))
 (segment (start 142.485 93.675) (end 146.71 97.9) (width 0.2) (layer "F.Cu") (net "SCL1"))
 (segment (start 146.71 97.9) (end 152.46 97.9) (width 0.2) (layer "F.Cu") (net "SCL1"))
 (segment (start 146.18 91.67) (end 146.18 92.354899) (width 0.2) (layer "F.Cu") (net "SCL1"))
 (segment (start 146.18 92.354899) (end 145.365 93.169899) (width 0.2) (layer "F.Cu") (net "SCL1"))
 (segment (start 145.365 93.169899) (end 142.990101 93.169899) (width 0.2) (layer "F.Cu") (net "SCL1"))
 (segment (start 152.4875 102.8675) (end 152.49 102.87) (width 0.2) (layer "F.Cu") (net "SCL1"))
 (segment (start 142.990101 93.169899) (end 142.485 93.675) (width 0.2) (layer "F.Cu") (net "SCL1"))
 (segment (start 142.46 103.59) (end 142.51 103.64) (width 0.2) (layer "F.Cu") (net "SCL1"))
 (segment (start 152.4875 102.0575) (end 152.4875 102.8675) (width 0.2) (layer "F.Cu") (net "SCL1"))
 (segment (start 142.485 93.675) (end 142.38 93.78) (width 0.2) (layer "F.Cu") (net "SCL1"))
 (via (at 141.13 103.59) (size 0.6) (drill 0.3) (layers "F.Cu" "B.Cu") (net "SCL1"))
 (via (at 152.49 102.87) (size 0.6) (drill 0.3) (layers "F.Cu" "B.Cu") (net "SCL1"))
 (via (at 141.6 94.56) (size 0.6) (drill 0.3) (layers "F.Cu" "B.Cu") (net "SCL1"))
 (via (at 152.46 97.9) (size 0.6) (drill 0.3) (layers "F.Cu" "B.Cu") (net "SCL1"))
 (segment (start 152.63 102.73) (end 152.49 102.87) (width 0.2) (layer "B.Cu") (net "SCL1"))
 (segment (start 152.63 98.07) (end 152.63 102.73) (width 0.2) (layer "B.Cu") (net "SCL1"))
 (segment (start 152.46 97.9) (end 152.63 98.07) (width 0.2) (layer "B.Cu") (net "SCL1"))
 (segment (start 141.6 94.56) (end 141.13 95.03) (width 0.2) (layer "B.Cu") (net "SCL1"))
 (segment (start 141.13 97.41) (end 141.13 103.59) (width 0.2) (layer "B.Cu") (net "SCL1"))
 (segment (start 141.13 95.03) (end 141.13 97.41) (width 0.2) (layer "B.Cu") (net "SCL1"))
 (segment (start 146.080268 104.59) (end 145.02 105.650268) (width 0.2) (layer "F.Cu") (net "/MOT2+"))
 (segment (start 146.81 104.64) (end 146.84 104.61) (width 0.2) (layer "F.Cu") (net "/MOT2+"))
 (segment (start 146.84 104.59) (end 146.080268 104.59) (width 0.2) (layer "F.Cu") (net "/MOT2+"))
 (segment (start 145.02 105.650268) (end 145.02 109.97) (width 0.2) (layer "F.Cu") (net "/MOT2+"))
 (segment (start 146.84 104.61) (end 146.84 104.59) (width 0.2) (layer "F.Cu") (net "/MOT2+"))
 (segment (start 142.03 102.66) (end 142.51 103.14) (width 0.2) (layer "F.Cu") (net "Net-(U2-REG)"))
 (segment (start 142.03 101.08) (end 142.03 102.66) (width 0.2) (layer "F.Cu") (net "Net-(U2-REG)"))
 (segment (start 151.705 107.46) (end 150.77 106.525) (width 0.2) (layer "F.Cu") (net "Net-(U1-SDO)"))
 (segment (start 150.77 102.3125) (end 150.8625 102.22) (width 0.2) (layer "F.Cu") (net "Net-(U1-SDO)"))
 (segment (start 150.77 106.525) (end 150.77 102.3125) (width 0.2) (layer "F.Cu") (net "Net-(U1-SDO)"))
 (segment (start 150.8625 102.22) (end 151.325 102.22) (width 0.2) (layer "F.Cu") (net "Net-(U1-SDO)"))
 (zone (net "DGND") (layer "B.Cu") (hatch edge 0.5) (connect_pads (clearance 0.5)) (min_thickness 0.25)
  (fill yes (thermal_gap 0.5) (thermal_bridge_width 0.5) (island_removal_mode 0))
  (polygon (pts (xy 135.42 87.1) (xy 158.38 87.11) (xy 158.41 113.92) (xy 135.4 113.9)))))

